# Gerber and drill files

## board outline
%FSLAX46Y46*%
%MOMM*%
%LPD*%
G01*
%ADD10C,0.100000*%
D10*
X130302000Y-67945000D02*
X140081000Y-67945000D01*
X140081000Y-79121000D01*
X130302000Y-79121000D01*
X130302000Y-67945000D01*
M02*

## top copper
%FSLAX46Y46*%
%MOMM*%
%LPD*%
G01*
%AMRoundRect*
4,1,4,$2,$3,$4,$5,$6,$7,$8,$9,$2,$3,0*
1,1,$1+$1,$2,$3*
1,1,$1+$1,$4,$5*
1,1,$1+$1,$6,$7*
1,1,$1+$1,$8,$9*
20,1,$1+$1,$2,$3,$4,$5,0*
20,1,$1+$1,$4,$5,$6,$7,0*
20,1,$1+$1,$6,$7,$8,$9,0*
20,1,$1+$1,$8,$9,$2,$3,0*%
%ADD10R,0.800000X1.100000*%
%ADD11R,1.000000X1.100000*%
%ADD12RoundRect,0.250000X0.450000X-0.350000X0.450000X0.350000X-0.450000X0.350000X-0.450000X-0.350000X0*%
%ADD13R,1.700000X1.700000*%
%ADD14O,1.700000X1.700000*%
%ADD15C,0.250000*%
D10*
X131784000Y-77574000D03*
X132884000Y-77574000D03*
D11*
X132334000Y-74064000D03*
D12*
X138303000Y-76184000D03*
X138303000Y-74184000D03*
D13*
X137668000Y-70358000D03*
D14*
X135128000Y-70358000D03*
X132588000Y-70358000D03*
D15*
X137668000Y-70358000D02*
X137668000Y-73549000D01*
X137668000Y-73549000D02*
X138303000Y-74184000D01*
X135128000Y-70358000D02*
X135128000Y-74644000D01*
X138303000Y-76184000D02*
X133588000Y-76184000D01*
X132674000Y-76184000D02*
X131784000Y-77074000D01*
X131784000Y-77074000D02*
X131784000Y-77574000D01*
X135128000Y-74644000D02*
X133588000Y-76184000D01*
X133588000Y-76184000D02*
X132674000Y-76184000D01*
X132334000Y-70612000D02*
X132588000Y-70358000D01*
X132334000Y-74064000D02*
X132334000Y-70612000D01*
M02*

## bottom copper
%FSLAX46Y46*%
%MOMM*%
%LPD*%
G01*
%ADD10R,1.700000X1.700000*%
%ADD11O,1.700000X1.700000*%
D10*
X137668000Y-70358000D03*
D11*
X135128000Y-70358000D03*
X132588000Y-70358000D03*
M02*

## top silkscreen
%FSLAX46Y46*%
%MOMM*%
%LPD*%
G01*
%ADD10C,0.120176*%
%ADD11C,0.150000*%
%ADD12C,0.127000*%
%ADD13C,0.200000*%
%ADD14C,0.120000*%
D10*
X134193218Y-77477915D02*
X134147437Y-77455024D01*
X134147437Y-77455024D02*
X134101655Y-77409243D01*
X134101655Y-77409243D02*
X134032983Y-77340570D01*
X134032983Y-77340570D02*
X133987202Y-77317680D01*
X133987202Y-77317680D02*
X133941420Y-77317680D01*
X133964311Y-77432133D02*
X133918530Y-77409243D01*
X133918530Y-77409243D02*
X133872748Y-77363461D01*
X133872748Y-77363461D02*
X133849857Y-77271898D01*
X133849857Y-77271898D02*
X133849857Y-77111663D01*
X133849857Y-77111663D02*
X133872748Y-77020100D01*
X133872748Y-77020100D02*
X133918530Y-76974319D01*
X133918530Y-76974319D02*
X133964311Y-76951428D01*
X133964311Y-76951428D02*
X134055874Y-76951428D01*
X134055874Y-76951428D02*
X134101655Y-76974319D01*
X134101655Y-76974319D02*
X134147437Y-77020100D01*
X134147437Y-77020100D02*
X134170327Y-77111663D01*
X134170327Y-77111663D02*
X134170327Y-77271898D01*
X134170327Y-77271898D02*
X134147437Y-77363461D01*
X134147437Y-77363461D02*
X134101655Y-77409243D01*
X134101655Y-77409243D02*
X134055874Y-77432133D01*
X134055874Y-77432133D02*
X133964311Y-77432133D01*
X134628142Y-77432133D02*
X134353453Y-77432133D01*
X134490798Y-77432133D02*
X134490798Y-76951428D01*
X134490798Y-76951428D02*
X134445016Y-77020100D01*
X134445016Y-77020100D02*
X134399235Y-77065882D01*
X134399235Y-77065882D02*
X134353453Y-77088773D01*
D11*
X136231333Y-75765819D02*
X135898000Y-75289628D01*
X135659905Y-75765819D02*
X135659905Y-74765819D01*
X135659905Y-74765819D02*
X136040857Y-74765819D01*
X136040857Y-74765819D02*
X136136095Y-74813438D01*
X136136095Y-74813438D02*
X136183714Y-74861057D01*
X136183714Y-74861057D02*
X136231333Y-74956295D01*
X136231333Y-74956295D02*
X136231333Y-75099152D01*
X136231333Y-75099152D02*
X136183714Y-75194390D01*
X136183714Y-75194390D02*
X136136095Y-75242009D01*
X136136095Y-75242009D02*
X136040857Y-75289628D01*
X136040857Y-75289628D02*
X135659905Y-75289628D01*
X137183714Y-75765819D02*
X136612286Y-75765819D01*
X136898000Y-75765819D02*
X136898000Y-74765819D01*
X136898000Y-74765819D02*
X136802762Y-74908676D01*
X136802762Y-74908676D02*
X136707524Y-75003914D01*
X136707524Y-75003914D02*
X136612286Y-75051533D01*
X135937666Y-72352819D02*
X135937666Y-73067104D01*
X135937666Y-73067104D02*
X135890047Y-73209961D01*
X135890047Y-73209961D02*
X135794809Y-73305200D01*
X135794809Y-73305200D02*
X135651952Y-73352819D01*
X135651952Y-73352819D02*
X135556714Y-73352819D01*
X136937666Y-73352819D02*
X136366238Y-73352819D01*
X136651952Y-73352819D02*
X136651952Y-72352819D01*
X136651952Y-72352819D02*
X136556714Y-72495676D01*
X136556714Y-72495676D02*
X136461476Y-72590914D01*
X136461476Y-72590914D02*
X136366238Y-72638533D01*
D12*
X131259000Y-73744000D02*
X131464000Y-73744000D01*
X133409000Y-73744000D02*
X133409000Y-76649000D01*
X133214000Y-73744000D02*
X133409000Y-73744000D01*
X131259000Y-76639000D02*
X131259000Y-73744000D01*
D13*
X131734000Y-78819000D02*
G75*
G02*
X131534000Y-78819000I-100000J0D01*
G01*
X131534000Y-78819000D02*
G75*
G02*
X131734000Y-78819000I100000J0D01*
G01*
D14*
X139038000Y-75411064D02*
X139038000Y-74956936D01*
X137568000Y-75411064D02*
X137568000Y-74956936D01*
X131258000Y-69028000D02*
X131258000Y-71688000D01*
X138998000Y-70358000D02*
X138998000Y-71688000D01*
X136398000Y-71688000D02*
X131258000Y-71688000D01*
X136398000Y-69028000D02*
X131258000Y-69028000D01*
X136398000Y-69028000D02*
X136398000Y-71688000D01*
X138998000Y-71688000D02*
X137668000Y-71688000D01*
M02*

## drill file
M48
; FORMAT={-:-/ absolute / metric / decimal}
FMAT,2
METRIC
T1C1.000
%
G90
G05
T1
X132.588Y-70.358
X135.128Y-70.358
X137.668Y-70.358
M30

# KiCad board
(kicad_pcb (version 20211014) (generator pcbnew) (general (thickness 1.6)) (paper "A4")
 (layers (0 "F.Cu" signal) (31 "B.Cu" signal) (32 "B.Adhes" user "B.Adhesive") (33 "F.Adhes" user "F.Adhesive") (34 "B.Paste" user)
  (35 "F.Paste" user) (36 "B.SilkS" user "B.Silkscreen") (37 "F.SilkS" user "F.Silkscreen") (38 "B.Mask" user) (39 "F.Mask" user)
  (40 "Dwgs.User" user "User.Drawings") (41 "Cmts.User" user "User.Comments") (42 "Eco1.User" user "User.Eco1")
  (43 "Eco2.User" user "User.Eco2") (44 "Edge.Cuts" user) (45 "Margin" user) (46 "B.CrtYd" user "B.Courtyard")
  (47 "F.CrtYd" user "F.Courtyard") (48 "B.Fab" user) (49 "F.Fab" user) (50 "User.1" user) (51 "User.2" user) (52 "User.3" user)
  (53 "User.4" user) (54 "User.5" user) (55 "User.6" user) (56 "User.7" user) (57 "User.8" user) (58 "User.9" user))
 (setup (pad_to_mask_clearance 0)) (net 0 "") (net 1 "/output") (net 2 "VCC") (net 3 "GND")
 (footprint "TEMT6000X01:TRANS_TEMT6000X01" (layer "F.Cu") (at 132.334 75.819 90)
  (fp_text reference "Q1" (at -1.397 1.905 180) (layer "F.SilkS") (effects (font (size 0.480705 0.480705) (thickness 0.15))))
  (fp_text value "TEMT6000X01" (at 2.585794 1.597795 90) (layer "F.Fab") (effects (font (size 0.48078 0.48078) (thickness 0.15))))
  (fp_line (start 2.075 -1.075) (end 2.075 -0.87) (layer "F.SilkS") (width 0.127))
  (fp_line (start 2.075 1.075) (end -0.83 1.075) (layer "F.SilkS") (width 0.127))
  (fp_line (start 2.075 0.88) (end 2.075 1.075) (layer "F.SilkS") (width 0.127))
  (fp_line (start -0.82 -1.075) (end 2.075 -1.075) (layer "F.SilkS") (width 0.127))
  (fp_circle (center -3 -0.7) (end -2.9 -0.7) (layer "F.SilkS") (width 0.2) (fill none))
  (pad "1" smd rect locked (at -1.755 -0.55 90) (size 1.1 0.8) (layers "F.Cu" "F.Paste" "F.Mask") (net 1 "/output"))
  (pad "2" smd rect locked (at -1.755 0.55 90) (size 1.1 0.8) (layers "F.Cu" "F.Paste" "F.Mask"))
  (pad "3" smd rect locked (at 1.755 0 90) (size 1.1 1) (layers "F.Cu" "F.Paste" "F.Mask") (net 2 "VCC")))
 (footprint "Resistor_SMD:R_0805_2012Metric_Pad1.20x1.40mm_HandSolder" (layer "F.Cu") (at 138.303 75.184 90)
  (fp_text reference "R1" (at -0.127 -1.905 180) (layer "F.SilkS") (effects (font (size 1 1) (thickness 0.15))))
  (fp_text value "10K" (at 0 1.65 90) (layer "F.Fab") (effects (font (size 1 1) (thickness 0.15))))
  (fp_line (start -0.227064 0.735) (end 0.227064 0.735) (layer "F.SilkS") (width 0.12))
  (fp_line (start -0.227064 -0.735) (end 0.227064 -0.735) (layer "F.SilkS") (width 0.12))
  (pad "1" smd roundrect (at -1 0 90) (size 1.2 1.4) (layers "F.Cu" "F.Paste" "F.Mask") (roundrect_rratio 0.208333) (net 1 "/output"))
  (pad "2" smd roundrect (at 1 0 90) (size 1.2 1.4) (layers "F.Cu" "F.Paste" "F.Mask") (roundrect_rratio 0.208333) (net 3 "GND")))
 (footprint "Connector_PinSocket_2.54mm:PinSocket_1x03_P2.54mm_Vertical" (layer "F.Cu") (at 137.668 70.358 -90)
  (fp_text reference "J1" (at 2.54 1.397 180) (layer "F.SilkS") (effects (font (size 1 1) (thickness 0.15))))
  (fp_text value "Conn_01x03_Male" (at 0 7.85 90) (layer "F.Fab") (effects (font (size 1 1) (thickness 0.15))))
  (fp_line (start -1.33 6.41) (end 1.33 6.41) (layer "F.SilkS") (width 0.12))
  (fp_line (start 0 -1.33) (end 1.33 -1.33) (layer "F.SilkS") (width 0.12))
  (fp_line (start 1.33 1.27) (end 1.33 6.41) (layer "F.SilkS") (width 0.12))
  (fp_line (start -1.33 1.27) (end -1.33 6.41) (layer "F.SilkS") (width 0.12))
  (fp_line (start -1.33 1.27) (end 1.33 1.27) (layer "F.SilkS") (width 0.12))
  (fp_line (start 1.33 -1.33) (end 1.33 0) (layer "F.SilkS") (width 0.12))
  (pad "1" thru_hole rect (at 0 0 270) (size 1.7 1.7) (drill 1) (layers *.Cu *.Mask) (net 3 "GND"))
  (pad "2" thru_hole oval (at 0 2.54 270) (size 1.7 1.7) (drill 1) (layers *.Cu *.Mask) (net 1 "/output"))
  (pad "3" thru_hole oval (at 0 5.08 270) (size 1.7 1.7) (drill 1) (layers *.Cu *.Mask) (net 2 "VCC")))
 (gr_rect (start 130.302 67.945) (end 140.081 79.121) (layer "Edge.Cuts") (width 0.1) (fill none))
 (segment (start 137.668 70.358) (end 137.668 73.549) (width 0.25) (layer "F.Cu") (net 3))
 (segment (start 137.668 73.549) (end 138.303 74.184) (width 0.25) (layer "F.Cu") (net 3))
 (segment (start 135.128 70.358) (end 135.128 74.644) (width 0.25) (layer "F.Cu") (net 1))
 (segment (start 138.303 76.184) (end 133.588 76.184) (width 0.25) (layer "F.Cu") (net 1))
 (segment (start 132.674 76.184) (end 131.784 77.074) (width 0.25) (layer "F.Cu") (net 1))
 (segment (start 131.784 77.074) (end 131.784 77.574) (width 0.25) (layer "F.Cu") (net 1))
 (segment (start 135.128 74.644) (end 133.588 76.184) (width 0.25) (layer "F.Cu") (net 1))
 (segment (start 133.588 76.184) (end 132.674 76.184) (width 0.25) (layer "F.Cu") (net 1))
 (segment (start 132.334 70.612) (end 132.588 70.358) (width 0.25) (layer "F.Cu") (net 2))
 (segment (start 132.334 74.064) (end 132.334 70.612) (width 0.25) (layer "F.Cu") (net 2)))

